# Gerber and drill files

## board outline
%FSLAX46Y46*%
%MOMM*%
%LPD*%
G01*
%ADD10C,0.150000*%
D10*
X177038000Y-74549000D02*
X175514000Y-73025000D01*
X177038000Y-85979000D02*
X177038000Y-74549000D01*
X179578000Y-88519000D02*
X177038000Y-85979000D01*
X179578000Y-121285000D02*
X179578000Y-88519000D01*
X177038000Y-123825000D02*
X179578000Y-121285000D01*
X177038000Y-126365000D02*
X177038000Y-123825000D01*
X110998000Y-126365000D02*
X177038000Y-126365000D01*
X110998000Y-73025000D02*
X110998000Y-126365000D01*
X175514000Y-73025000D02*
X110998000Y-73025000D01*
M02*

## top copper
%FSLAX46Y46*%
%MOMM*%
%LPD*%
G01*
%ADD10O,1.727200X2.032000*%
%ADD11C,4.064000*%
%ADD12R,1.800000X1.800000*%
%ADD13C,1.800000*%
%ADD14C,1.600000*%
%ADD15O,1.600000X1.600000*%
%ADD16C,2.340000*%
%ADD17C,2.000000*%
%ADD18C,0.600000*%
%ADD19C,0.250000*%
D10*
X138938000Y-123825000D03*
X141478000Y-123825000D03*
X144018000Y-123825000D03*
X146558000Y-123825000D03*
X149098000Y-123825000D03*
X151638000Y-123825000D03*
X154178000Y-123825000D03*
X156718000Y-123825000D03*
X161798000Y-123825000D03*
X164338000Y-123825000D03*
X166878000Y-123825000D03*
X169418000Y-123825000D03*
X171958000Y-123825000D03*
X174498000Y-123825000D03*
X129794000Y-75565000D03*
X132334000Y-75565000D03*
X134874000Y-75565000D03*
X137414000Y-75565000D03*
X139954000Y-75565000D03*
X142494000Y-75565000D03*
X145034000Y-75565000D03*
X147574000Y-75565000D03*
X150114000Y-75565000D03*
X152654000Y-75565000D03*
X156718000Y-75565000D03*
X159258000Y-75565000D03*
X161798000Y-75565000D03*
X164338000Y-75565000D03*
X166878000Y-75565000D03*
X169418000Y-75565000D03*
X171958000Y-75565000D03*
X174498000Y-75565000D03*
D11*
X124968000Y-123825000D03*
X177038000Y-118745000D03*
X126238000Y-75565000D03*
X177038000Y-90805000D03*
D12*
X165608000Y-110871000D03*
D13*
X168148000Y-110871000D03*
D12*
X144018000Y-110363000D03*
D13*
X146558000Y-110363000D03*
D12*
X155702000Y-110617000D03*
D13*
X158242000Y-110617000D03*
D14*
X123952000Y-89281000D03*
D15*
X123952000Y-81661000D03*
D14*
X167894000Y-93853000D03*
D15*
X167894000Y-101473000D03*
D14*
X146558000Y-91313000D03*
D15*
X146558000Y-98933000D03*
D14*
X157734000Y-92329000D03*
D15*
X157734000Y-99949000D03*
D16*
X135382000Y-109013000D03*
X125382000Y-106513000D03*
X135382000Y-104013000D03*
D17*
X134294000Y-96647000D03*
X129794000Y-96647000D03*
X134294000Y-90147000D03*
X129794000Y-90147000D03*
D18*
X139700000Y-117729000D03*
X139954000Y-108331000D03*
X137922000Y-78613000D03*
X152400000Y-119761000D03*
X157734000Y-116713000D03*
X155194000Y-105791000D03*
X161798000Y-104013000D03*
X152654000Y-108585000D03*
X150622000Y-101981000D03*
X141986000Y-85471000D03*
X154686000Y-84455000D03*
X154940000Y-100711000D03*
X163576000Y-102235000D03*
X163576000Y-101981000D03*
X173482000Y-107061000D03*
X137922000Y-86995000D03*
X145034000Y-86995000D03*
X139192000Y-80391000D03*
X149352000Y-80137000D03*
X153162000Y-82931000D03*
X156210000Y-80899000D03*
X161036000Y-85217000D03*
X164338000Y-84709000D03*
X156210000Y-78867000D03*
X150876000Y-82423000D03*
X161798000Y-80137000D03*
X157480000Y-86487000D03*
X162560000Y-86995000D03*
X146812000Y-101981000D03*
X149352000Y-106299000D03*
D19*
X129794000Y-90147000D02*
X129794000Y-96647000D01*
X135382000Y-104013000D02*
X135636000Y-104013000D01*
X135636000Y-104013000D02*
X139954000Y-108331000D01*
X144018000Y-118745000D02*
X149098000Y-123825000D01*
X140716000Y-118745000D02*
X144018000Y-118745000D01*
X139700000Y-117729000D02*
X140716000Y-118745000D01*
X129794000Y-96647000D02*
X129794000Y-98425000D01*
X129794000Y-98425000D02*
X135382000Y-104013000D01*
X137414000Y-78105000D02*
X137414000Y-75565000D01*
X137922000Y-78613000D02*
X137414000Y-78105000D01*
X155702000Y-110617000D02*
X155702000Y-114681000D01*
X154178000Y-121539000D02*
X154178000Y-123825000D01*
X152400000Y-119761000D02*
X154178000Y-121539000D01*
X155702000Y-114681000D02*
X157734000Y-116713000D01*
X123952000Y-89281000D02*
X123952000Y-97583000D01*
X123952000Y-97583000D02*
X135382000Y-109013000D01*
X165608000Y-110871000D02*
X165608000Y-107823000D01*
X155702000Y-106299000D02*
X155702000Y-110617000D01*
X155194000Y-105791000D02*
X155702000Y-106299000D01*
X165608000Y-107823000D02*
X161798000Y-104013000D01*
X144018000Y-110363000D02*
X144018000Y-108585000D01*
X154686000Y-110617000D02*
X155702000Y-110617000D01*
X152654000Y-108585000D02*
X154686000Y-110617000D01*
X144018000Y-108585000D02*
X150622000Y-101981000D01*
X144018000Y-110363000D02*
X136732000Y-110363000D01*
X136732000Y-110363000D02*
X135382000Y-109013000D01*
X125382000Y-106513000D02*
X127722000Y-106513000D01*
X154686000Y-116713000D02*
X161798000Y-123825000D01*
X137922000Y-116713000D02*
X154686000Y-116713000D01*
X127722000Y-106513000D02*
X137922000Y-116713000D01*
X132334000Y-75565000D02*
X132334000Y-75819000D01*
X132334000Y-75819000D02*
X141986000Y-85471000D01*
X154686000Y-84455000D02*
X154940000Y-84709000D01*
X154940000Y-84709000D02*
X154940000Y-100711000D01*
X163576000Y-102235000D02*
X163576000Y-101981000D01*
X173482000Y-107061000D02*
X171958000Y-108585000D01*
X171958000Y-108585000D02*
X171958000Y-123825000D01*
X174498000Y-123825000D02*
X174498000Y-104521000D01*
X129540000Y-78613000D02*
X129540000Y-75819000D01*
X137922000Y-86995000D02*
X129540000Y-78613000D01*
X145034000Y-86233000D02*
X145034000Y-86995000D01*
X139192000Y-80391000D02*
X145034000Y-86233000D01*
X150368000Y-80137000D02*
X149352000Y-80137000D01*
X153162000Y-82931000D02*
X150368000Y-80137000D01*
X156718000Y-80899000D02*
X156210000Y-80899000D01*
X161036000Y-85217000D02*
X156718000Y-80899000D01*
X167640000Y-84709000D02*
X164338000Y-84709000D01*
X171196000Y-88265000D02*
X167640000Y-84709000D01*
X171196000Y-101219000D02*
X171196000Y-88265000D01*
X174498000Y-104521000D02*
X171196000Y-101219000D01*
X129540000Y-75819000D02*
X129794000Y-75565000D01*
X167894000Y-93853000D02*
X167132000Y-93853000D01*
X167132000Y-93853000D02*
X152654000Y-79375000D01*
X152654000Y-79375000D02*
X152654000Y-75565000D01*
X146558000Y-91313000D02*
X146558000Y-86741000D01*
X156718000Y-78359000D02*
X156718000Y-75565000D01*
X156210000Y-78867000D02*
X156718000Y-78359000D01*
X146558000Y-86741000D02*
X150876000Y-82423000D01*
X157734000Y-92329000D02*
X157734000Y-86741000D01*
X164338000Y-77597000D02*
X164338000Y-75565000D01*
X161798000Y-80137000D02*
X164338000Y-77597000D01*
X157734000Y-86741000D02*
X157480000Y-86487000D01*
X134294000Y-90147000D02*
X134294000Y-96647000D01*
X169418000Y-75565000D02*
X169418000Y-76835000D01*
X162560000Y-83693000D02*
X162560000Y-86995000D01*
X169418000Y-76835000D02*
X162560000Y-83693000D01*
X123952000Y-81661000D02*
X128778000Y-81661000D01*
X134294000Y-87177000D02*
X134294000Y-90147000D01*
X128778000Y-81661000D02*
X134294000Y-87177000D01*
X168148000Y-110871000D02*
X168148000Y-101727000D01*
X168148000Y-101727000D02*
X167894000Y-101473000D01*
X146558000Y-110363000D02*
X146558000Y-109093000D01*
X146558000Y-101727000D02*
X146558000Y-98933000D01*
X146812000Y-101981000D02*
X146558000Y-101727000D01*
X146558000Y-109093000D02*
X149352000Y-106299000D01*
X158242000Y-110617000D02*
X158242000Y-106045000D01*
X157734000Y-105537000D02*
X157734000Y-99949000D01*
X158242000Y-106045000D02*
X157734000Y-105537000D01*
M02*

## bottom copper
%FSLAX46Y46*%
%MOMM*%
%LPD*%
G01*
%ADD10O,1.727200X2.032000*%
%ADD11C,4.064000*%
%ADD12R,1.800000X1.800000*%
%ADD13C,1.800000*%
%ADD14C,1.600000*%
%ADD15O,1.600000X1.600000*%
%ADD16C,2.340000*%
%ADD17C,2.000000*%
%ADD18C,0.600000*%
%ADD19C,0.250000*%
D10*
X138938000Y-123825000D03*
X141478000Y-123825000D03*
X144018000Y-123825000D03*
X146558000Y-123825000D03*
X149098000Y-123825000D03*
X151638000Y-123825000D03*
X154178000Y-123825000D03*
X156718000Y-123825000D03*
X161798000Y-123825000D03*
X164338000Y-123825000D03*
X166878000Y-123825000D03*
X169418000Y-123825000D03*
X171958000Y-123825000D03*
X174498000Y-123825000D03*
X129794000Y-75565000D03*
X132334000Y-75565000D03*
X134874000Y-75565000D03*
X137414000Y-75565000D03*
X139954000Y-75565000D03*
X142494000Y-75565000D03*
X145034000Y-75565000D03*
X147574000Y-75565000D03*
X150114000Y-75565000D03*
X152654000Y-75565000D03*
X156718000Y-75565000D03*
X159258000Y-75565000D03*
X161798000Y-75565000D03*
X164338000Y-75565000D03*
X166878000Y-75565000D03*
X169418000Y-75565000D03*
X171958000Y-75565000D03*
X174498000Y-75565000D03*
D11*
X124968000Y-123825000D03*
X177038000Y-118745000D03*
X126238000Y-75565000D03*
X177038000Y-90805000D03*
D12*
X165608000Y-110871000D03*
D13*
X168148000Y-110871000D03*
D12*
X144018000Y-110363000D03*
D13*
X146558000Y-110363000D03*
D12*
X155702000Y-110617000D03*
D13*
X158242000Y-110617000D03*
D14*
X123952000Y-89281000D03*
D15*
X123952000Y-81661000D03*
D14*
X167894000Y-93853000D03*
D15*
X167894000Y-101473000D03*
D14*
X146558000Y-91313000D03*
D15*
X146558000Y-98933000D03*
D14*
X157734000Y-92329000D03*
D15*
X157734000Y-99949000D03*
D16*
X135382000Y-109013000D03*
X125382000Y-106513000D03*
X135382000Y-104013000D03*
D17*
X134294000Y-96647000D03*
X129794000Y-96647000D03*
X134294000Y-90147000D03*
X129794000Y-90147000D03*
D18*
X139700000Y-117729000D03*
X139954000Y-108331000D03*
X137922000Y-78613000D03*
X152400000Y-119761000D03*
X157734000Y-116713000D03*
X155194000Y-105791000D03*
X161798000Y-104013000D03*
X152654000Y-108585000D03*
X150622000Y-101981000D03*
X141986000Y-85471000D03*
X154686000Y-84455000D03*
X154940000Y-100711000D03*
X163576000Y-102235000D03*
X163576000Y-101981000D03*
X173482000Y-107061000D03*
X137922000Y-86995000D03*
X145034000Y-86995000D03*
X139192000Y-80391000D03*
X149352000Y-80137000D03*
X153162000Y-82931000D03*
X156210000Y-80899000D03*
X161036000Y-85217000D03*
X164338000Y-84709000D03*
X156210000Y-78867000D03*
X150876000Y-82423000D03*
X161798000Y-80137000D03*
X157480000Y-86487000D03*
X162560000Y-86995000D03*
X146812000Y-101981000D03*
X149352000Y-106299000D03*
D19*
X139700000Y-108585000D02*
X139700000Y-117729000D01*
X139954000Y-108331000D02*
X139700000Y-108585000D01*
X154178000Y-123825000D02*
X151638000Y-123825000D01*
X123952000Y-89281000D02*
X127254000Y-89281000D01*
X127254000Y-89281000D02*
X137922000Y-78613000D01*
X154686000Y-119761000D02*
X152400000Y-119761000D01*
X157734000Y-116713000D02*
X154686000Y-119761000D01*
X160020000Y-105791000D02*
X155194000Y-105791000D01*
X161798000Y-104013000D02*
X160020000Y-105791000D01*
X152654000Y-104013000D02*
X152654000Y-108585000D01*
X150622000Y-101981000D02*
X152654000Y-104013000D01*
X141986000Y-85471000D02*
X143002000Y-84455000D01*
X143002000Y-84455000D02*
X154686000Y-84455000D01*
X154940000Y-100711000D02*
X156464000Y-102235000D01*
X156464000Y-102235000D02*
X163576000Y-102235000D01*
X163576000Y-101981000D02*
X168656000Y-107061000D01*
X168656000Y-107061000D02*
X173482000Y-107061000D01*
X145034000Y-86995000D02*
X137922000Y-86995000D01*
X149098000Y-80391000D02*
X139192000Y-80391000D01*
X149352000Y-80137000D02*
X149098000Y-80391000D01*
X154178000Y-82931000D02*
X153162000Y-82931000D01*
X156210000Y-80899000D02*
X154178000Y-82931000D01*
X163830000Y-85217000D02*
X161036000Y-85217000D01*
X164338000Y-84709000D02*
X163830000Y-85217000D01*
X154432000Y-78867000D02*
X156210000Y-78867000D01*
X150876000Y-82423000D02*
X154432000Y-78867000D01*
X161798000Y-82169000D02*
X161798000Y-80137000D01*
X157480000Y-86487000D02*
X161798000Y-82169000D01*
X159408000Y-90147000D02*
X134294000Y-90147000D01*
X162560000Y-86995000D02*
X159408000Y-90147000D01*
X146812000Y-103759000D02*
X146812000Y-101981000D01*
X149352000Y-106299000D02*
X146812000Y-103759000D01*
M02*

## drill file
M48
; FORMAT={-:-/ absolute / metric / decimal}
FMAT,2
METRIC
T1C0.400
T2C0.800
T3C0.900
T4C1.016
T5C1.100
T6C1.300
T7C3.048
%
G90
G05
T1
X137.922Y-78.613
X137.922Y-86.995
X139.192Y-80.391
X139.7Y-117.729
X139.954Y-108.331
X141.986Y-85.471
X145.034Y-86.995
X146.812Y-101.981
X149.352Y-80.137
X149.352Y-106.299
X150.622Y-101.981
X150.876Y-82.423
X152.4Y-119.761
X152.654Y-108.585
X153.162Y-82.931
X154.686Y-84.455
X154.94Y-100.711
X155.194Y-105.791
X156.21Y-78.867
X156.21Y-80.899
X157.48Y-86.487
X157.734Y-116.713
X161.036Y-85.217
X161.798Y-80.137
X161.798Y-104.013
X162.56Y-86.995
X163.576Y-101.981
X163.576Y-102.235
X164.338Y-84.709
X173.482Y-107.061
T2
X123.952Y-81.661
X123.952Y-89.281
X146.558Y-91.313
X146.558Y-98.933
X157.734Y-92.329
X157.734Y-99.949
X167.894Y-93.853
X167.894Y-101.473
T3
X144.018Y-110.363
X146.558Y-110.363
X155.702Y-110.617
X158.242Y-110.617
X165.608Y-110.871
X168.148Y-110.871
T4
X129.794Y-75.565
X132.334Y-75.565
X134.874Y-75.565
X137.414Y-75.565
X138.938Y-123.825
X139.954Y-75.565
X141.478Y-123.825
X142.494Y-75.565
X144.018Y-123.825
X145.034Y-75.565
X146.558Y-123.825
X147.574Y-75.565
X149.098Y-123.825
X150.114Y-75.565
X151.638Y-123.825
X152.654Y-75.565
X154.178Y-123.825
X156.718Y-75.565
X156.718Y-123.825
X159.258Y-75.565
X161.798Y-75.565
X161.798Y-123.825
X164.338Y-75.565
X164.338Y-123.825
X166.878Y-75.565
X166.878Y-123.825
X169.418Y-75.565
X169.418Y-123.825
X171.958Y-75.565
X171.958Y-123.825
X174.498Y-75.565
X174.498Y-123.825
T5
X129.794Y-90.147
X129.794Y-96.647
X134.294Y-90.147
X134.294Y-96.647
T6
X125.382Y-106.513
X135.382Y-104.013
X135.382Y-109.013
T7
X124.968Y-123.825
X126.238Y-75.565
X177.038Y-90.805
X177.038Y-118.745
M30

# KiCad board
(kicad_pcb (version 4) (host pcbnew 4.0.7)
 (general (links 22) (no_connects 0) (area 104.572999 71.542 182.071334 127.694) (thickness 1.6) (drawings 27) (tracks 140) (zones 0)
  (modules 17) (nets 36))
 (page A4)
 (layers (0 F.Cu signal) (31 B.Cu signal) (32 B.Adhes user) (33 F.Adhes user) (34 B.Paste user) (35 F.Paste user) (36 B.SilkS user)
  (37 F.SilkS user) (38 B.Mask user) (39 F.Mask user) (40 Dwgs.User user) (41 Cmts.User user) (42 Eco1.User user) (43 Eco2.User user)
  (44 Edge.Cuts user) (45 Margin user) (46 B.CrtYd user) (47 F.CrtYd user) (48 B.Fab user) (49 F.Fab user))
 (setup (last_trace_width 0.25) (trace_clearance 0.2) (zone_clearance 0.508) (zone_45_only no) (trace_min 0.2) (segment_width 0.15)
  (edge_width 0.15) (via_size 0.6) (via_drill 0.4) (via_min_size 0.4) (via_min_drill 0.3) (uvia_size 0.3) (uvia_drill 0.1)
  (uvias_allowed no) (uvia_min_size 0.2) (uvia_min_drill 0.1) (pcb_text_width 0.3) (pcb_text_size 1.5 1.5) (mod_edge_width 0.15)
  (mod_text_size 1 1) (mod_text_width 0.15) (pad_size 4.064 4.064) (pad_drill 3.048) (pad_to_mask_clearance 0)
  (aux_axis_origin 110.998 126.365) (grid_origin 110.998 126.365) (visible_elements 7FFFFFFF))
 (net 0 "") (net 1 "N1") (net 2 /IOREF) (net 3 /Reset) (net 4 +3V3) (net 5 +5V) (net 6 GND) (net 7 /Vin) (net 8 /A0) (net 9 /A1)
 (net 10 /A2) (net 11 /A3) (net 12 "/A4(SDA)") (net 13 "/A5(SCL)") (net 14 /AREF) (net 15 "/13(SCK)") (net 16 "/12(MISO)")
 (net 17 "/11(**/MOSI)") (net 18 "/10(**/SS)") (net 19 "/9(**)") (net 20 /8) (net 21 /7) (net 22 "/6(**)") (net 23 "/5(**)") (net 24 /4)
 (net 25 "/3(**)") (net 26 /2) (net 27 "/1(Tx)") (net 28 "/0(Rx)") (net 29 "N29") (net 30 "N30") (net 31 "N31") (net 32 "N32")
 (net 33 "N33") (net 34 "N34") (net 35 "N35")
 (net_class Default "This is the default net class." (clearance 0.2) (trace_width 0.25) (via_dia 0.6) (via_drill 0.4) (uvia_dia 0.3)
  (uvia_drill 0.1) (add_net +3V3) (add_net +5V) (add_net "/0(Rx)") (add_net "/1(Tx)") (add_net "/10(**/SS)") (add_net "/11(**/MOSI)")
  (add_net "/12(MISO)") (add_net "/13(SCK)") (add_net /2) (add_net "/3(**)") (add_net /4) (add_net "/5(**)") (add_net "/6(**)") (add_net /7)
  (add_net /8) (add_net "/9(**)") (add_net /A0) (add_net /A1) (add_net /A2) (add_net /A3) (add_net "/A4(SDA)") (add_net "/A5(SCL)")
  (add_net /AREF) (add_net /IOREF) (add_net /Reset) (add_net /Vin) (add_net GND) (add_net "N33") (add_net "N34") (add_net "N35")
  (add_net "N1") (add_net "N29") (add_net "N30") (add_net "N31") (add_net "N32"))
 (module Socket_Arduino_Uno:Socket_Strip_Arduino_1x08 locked (layer F.Cu) (at 138.938 123.825)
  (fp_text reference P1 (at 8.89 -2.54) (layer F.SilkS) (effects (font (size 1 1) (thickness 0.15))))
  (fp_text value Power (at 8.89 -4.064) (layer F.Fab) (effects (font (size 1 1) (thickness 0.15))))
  (pad 1 thru_hole oval (at 0 0) (size 1.7272 2.032) (drill 1.016) (layers *.Cu *.Mask F.SilkS) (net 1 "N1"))
  (pad 2 thru_hole oval (at 2.54 0) (size 1.7272 2.032) (drill 1.016) (layers *.Cu *.Mask F.SilkS) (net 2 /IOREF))
  (pad 3 thru_hole oval (at 5.08 0) (size 1.7272 2.032) (drill 1.016) (layers *.Cu *.Mask F.SilkS) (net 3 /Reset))
  (pad 4 thru_hole oval (at 7.62 0) (size 1.7272 2.032) (drill 1.016) (layers *.Cu *.Mask F.SilkS) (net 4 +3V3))
  (pad 5 thru_hole oval (at 10.16 0) (size 1.7272 2.032) (drill 1.016) (layers *.Cu *.Mask F.SilkS) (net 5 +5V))
  (pad 6 thru_hole oval (at 12.7 0) (size 1.7272 2.032) (drill 1.016) (layers *.Cu *.Mask F.SilkS) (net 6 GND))
  (pad 7 thru_hole oval (at 15.24 0) (size 1.7272 2.032) (drill 1.016) (layers *.Cu *.Mask F.SilkS) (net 6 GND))
  (pad 8 thru_hole oval (at 17.78 0) (size 1.7272 2.032) (drill 1.016) (layers *.Cu *.Mask F.SilkS) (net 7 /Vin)))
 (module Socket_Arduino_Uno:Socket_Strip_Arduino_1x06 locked (layer F.Cu) (at 161.798 123.825)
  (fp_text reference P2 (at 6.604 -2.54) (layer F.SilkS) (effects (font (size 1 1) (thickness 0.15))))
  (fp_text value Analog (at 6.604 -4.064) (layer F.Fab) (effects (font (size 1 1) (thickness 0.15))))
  (pad 1 thru_hole oval (at 0 0) (size 1.7272 2.032) (drill 1.016) (layers *.Cu *.Mask F.SilkS) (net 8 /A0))
  (pad 2 thru_hole oval (at 2.54 0) (size 1.7272 2.032) (drill 1.016) (layers *.Cu *.Mask F.SilkS) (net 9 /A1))
  (pad 3 thru_hole oval (at 5.08 0) (size 1.7272 2.032) (drill 1.016) (layers *.Cu *.Mask F.SilkS) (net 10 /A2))
  (pad 4 thru_hole oval (at 7.62 0) (size 1.7272 2.032) (drill 1.016) (layers *.Cu *.Mask F.SilkS) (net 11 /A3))
  (pad 5 thru_hole oval (at 10.16 0) (size 1.7272 2.032) (drill 1.016) (layers *.Cu *.Mask F.SilkS) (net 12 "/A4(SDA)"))
  (pad 6 thru_hole oval (at 12.7 0) (size 1.7272 2.032) (drill 1.016) (layers *.Cu *.Mask F.SilkS) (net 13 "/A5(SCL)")))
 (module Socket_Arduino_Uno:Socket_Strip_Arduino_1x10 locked (layer F.Cu) (at 129.794 75.565)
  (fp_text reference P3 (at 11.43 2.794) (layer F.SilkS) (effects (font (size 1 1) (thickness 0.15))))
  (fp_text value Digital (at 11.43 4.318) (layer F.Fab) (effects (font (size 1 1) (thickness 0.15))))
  (pad 1 thru_hole oval (at 0 0) (size 1.7272 2.032) (drill 1.016) (layers *.Cu *.Mask F.SilkS) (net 13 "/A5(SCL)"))
  (pad 2 thru_hole oval (at 2.54 0) (size 1.7272 2.032) (drill 1.016) (layers *.Cu *.Mask F.SilkS) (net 12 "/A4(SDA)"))
  (pad 3 thru_hole oval (at 5.08 0) (size 1.7272 2.032) (drill 1.016) (layers *.Cu *.Mask F.SilkS) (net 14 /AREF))
  (pad 4 thru_hole oval (at 7.62 0) (size 1.7272 2.032) (drill 1.016) (layers *.Cu *.Mask F.SilkS) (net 6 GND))
  (pad 5 thru_hole oval (at 10.16 0) (size 1.7272 2.032) (drill 1.016) (layers *.Cu *.Mask F.SilkS) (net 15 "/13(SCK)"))
  (pad 6 thru_hole oval (at 12.7 0) (size 1.7272 2.032) (drill 1.016) (layers *.Cu *.Mask F.SilkS) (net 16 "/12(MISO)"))
  (pad 7 thru_hole oval (at 15.24 0) (size 1.7272 2.032) (drill 1.016) (layers *.Cu *.Mask F.SilkS) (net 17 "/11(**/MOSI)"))
  (pad 8 thru_hole oval (at 17.78 0) (size 1.7272 2.032) (drill 1.016) (layers *.Cu *.Mask F.SilkS) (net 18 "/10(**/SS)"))
  (pad 9 thru_hole oval (at 20.32 0) (size 1.7272 2.032) (drill 1.016) (layers *.Cu *.Mask F.SilkS) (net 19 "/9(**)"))
  (pad 10 thru_hole oval (at 22.86 0) (size 1.7272 2.032) (drill 1.016) (layers *.Cu *.Mask F.SilkS) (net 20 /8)))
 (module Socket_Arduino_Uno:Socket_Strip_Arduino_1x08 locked (layer F.Cu) (at 156.718 75.565)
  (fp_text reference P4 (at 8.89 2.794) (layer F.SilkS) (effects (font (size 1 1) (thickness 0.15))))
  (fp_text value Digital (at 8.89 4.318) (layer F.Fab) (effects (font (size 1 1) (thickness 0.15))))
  (pad 1 thru_hole oval (at 0 0) (size 1.7272 2.032) (drill 1.016) (layers *.Cu *.Mask F.SilkS) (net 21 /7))
  (pad 2 thru_hole oval (at 2.54 0) (size 1.7272 2.032) (drill 1.016) (layers *.Cu *.Mask F.SilkS) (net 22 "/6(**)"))
  (pad 3 thru_hole oval (at 5.08 0) (size 1.7272 2.032) (drill 1.016) (layers *.Cu *.Mask F.SilkS) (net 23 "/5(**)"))
  (pad 4 thru_hole oval (at 7.62 0) (size 1.7272 2.032) (drill 1.016) (layers *.Cu *.Mask F.SilkS) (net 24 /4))
  (pad 5 thru_hole oval (at 10.16 0) (size 1.7272 2.032) (drill 1.016) (layers *.Cu *.Mask F.SilkS) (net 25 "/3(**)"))
  (pad 6 thru_hole oval (at 12.7 0) (size 1.7272 2.032) (drill 1.016) (layers *.Cu *.Mask F.SilkS) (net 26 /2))
  (pad 7 thru_hole oval (at 15.24 0) (size 1.7272 2.032) (drill 1.016) (layers *.Cu *.Mask F.SilkS) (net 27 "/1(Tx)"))
  (pad 8 thru_hole oval (at 17.78 0) (size 1.7272 2.032) (drill 1.016) (layers *.Cu *.Mask F.SilkS) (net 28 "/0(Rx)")))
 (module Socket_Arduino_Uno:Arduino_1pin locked (layer F.Cu) (at 124.968 123.825)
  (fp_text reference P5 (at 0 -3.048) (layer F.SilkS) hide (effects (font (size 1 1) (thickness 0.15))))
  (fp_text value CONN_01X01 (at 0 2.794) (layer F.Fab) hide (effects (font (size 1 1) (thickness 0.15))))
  (pad 1 thru_hole circle (at 0 0) (size 4.064 4.064) (drill 3.048) (layers *.Cu *.Mask F.SilkS) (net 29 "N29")))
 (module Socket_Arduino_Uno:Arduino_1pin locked (layer F.Cu) (at 177.038 118.745)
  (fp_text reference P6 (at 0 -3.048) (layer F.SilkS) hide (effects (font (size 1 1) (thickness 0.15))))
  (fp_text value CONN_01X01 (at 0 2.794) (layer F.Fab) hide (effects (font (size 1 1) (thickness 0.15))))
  (pad 1 thru_hole circle (at 0 0) (size 4.064 4.064) (drill 3.048) (layers *.Cu *.Mask F.SilkS) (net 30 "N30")))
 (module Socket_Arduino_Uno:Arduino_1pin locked (layer F.Cu) (at 126.238 75.565)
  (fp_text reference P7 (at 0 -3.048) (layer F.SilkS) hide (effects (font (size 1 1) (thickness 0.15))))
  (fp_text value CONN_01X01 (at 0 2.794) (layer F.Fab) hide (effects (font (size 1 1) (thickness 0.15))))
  (pad 1 thru_hole circle (at 0 0) (size 4.064 4.064) (drill 3.048) (layers *.Cu *.Mask F.SilkS) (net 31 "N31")))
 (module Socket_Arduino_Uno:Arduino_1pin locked (layer F.Cu) (at 177.038 90.805)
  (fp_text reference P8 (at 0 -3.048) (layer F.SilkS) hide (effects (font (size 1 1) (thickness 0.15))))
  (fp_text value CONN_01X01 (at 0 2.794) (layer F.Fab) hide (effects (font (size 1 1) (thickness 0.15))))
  (pad 1 thru_hole circle (at 0 0) (size 4.064 4.064) (drill 3.048) (layers *.Cu *.Mask F.SilkS) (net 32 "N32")))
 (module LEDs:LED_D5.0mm (layer F.Cu) (at 165.608 110.871)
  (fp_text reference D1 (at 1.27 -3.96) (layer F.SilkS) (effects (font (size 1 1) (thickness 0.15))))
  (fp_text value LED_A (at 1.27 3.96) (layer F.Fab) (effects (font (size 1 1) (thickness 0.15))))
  (pad 1 thru_hole rect (at 0 0) (size 1.8 1.8) (drill 0.9) (layers *.Cu *.Mask) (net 6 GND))
  (pad 2 thru_hole circle (at 2.54 0) (size 1.8 1.8) (drill 0.9) (layers *.Cu *.Mask) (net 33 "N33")))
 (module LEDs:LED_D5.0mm (layer F.Cu) (at 144.018 110.363)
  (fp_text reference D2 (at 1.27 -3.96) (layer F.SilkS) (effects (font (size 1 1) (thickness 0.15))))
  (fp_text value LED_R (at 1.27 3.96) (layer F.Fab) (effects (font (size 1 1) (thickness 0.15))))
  (pad 1 thru_hole rect (at 0 0) (size 1.8 1.8) (drill 0.9) (layers *.Cu *.Mask) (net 6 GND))
  (pad 2 thru_hole circle (at 2.54 0) (size 1.8 1.8) (drill 0.9) (layers *.Cu *.Mask) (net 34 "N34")))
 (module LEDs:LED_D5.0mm (layer F.Cu) (at 155.702 110.617)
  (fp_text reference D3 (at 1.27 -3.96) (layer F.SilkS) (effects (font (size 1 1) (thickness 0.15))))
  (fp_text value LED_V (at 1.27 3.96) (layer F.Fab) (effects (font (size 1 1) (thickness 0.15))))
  (pad 1 thru_hole rect (at 0 0) (size 1.8 1.8) (drill 0.9) (layers *.Cu *.Mask) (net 6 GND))
  (pad 2 thru_hole circle (at 2.54 0) (size 1.8 1.8) (drill 0.9) (layers *.Cu *.Mask) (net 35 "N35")))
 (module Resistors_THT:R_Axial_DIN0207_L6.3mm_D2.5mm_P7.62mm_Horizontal (layer F.Cu) (at 123.952 89.281 90)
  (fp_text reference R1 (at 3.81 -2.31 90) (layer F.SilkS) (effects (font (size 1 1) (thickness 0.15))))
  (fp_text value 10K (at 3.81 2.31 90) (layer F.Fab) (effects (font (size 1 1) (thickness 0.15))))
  (pad 1 thru_hole circle (at 0 0 90) (size 1.6 1.6) (drill 0.8) (layers *.Cu *.Mask) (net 6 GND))
  (pad 2 thru_hole oval (at 7.62 0 90) (size 1.6 1.6) (drill 0.8) (layers *.Cu *.Mask) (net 26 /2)))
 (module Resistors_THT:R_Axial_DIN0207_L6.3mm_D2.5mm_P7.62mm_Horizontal (layer F.Cu) (at 167.894 93.853 270)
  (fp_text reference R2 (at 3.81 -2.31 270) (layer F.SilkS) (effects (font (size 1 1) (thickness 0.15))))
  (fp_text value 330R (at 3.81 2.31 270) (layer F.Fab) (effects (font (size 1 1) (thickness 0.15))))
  (pad 1 thru_hole circle (at 0 0 270) (size 1.6 1.6) (drill 0.8) (layers *.Cu *.Mask) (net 20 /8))
  (pad 2 thru_hole oval (at 7.62 0 270) (size 1.6 1.6) (drill 0.8) (layers *.Cu *.Mask) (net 33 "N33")))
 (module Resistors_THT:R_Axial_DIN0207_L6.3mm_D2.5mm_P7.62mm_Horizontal (layer F.Cu) (at 146.558 91.313 270)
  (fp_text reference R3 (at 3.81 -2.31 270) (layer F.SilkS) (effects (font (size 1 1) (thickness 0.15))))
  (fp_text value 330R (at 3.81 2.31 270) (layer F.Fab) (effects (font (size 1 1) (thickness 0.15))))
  (pad 1 thru_hole circle (at 0 0 270) (size 1.6 1.6) (drill 0.8) (layers *.Cu *.Mask) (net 21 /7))
  (pad 2 thru_hole oval (at 7.62 0 270) (size 1.6 1.6) (drill 0.8) (layers *.Cu *.Mask) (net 34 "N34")))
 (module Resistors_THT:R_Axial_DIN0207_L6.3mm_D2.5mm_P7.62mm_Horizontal (layer F.Cu) (at 157.734 92.329 270)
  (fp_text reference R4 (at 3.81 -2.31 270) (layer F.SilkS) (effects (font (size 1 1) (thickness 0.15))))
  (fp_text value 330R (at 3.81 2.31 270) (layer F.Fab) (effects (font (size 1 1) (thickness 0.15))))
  (pad 1 thru_hole circle (at 0 0 270) (size 1.6 1.6) (drill 0.8) (layers *.Cu *.Mask) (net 24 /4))
  (pad 2 thru_hole oval (at 7.62 0 270) (size 1.6 1.6) (drill 0.8) (layers *.Cu *.Mask) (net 35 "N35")))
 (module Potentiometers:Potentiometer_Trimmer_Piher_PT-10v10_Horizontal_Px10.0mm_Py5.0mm (layer F.Cu) (at 135.382 104.013 180)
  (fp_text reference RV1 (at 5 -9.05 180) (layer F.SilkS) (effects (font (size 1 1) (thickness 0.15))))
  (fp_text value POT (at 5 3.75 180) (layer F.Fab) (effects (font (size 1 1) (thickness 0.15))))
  (pad 3 thru_hole circle (at 0 -5 180) (size 2.34 2.34) (drill 1.3) (layers *.Cu *.Mask) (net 6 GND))
  (pad 2 thru_hole circle (at 10 -2.5 180) (size 2.34 2.34) (drill 1.3) (layers *.Cu *.Mask) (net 8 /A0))
  (pad 1 thru_hole circle (at 0 0 180) (size 2.34 2.34) (drill 1.3) (layers *.Cu *.Mask) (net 5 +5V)))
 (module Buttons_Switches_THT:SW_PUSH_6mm (layer F.Cu) (at 129.794 96.647 90)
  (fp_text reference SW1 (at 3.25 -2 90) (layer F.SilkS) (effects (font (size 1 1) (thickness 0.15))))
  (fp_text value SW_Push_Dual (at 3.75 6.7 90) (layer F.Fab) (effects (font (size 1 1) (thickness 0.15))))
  (pad 2 thru_hole circle (at 0 4.5 180) (size 2 2) (drill 1.1) (layers *.Cu *.Mask) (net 26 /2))
  (pad 1 thru_hole circle (at 0 0 180) (size 2 2) (drill 1.1) (layers *.Cu *.Mask) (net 5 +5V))
  (pad 2 thru_hole circle (at 6.5 4.5 180) (size 2 2) (drill 1.1) (layers *.Cu *.Mask) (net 26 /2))
  (pad 1 thru_hole circle (at 6.5 0 180) (size 2 2) (drill 1.1) (layers *.Cu *.Mask) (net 5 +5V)))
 (gr_line (start 177.038 74.549) (end 175.514 73.025) (angle 90) (layer Edge.Cuts) (width 0.15))
 (gr_line (start 177.038 85.979) (end 177.038 74.549) (angle 90) (layer Edge.Cuts) (width 0.15))
 (gr_line (start 179.578 88.519) (end 177.038 85.979) (angle 90) (layer Edge.Cuts) (width 0.15))
 (gr_line (start 179.578 121.285) (end 179.578 88.519) (angle 90) (layer Edge.Cuts) (width 0.15))
 (gr_line (start 177.038 123.825) (end 179.578 121.285) (angle 90) (layer Edge.Cuts) (width 0.15))
 (gr_line (start 177.038 126.365) (end 177.038 123.825) (angle 90) (layer Edge.Cuts) (width 0.15))
 (gr_line (start 110.998 126.365) (end 177.038 126.365) (angle 90) (layer Edge.Cuts) (width 0.15))
 (gr_line (start 110.998 73.025) (end 110.998 126.365) (angle 90) (layer Edge.Cuts) (width 0.15))
 (gr_line (start 175.514 73.025) (end 110.998 73.025) (angle 90) (layer Edge.Cuts) (width 0.15))
 (segment (start 129.794 90.147) (end 129.794 96.647) (width 0.25) (layer F.Cu) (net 5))
 (segment (start 135.382 104.013) (end 135.636 104.013) (width 0.25) (layer F.Cu) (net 5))
 (segment (start 135.636 104.013) (end 139.954 108.331) (width 0.25) (layer F.Cu) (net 5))
 (segment (start 144.018 118.745) (end 149.098 123.825) (width 0.25) (layer F.Cu) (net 5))
 (segment (start 140.716 118.745) (end 144.018 118.745) (width 0.25) (layer F.Cu) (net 5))
 (segment (start 139.7 117.729) (end 140.716 118.745) (width 0.25) (layer F.Cu) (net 5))
 (via (at 139.7 117.729) (size 0.6) (drill 0.4) (layers F.Cu B.Cu) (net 5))
 (segment (start 139.7 108.585) (end 139.7 117.729) (width 0.25) (layer B.Cu) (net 5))
 (segment (start 139.954 108.331) (end 139.7 108.585) (width 0.25) (layer B.Cu) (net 5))
 (via (at 139.954 108.331) (size 0.6) (drill 0.4) (layers F.Cu B.Cu) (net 5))
 (segment (start 129.794 96.647) (end 129.794 98.425) (width 0.25) (layer F.Cu) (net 5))
 (segment (start 129.794 98.425) (end 135.382 104.013) (width 0.25) (layer F.Cu) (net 5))
 (segment (start 154.178 123.825) (end 151.638 123.825) (width 0.25) (layer B.Cu) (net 6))
 (segment (start 123.952 89.281) (end 127.254 89.281) (width 0.25) (layer B.Cu) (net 6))
 (segment (start 137.414 78.105) (end 137.414 75.565) (width 0.25) (layer F.Cu) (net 6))
 (segment (start 137.922 78.613) (end 137.414 78.105) (width 0.25) (layer F.Cu) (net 6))
 (via (at 137.922 78.613) (size 0.6) (drill 0.4) (layers F.Cu B.Cu) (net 6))
 (segment (start 127.254 89.281) (end 137.922 78.613) (width 0.25) (layer B.Cu) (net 6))
 (segment (start 155.702 110.617) (end 155.702 114.681) (width 0.25) (layer F.Cu) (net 6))
 (segment (start 154.178 121.539) (end 154.178 123.825) (width 0.25) (layer F.Cu) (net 6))
 (segment (start 152.4 119.761) (end 154.178 121.539) (width 0.25) (layer F.Cu) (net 6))
 (via (at 152.4 119.761) (size 0.6) (drill 0.4) (layers F.Cu B.Cu) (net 6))
 (segment (start 154.686 119.761) (end 152.4 119.761) (width 0.25) (layer B.Cu) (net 6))
 (segment (start 157.734 116.713) (end 154.686 119.761) (width 0.25) (layer B.Cu) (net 6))
 (via (at 157.734 116.713) (size 0.6) (drill 0.4) (layers F.Cu B.Cu) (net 6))
 (segment (start 155.702 114.681) (end 157.734 116.713) (width 0.25) (layer F.Cu) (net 6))
 (segment (start 123.952 89.281) (end 123.952 97.583) (width 0.25) (layer F.Cu) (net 6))
 (segment (start 123.952 97.583) (end 135.382 109.013) (width 0.25) (layer F.Cu) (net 6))
 (segment (start 165.608 110.871) (end 165.608 107.823) (width 0.25) (layer F.Cu) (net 6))
 (segment (start 155.702 106.299) (end 155.702 110.617) (width 0.25) (layer F.Cu) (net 6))
 (segment (start 155.194 105.791) (end 155.702 106.299) (width 0.25) (layer F.Cu) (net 6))
 (via (at 155.194 105.791) (size 0.6) (drill 0.4) (layers F.Cu B.Cu) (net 6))
 (segment (start 160.02 105.791) (end 155.194 105.791) (width 0.25) (layer B.Cu) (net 6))
 (segment (start 161.798 104.013) (end 160.02 105.791) (width 0.25) (layer B.Cu) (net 6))
 (via (at 161.798 104.013) (size 0.6) (drill 0.4) (layers F.Cu B.Cu) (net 6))
 (segment (start 165.608 107.823) (end 161.798 104.013) (width 0.25) (layer F.Cu) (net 6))
 (segment (start 144.018 110.363) (end 144.018 108.585) (width 0.25) (layer F.Cu) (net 6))
 (segment (start 154.686 110.617) (end 155.702 110.617) (width 0.25) (layer F.Cu) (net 6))
 (segment (start 152.654 108.585) (end 154.686 110.617) (width 0.25) (layer F.Cu) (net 6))
 (via (at 152.654 108.585) (size 0.6) (drill 0.4) (layers F.Cu B.Cu) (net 6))
 (segment (start 152.654 104.013) (end 152.654 108.585) (width 0.25) (layer B.Cu) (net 6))
 (segment (start 150.622 101.981) (end 152.654 104.013) (width 0.25) (layer B.Cu) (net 6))
 (via (at 150.622 101.981) (size 0.6) (drill 0.4) (layers F.Cu B.Cu) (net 6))
 (segment (start 144.018 108.585) (end 150.622 101.981) (width 0.25) (layer F.Cu) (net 6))
 (segment (start 144.018 110.363) (end 136.732 110.363) (width 0.25) (layer F.Cu) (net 6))
 (segment (start 136.732 110.363) (end 135.382 109.013) (width 0.25) (layer F.Cu) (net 6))
 (segment (start 125.382 106.513) (end 127.722 106.513) (width 0.25) (layer F.Cu) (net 8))
 (segment (start 154.686 116.713) (end 161.798 123.825) (width 0.25) (layer F.Cu) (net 8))
 (segment (start 137.922 116.713) (end 154.686 116.713) (width 0.25) (layer F.Cu) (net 8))
 (segment (start 127.722 106.513) (end 137.922 116.713) (width 0.25) (layer F.Cu) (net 8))
 (segment (start 132.334 75.565) (end 132.334 75.819) (width 0.25) (layer F.Cu) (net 12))
 (segment (start 132.334 75.819) (end 141.986 85.471) (width 0.25) (layer F.Cu) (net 12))
 (via (at 141.986 85.471) (size 0.6) (drill 0.4) (layers F.Cu B.Cu) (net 12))
 (segment (start 141.986 85.471) (end 143.002 84.455) (width 0.25) (layer B.Cu) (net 12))
 (segment (start 143.002 84.455) (end 154.686 84.455) (width 0.25) (layer B.Cu) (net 12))
 (via (at 154.686 84.455) (size 0.6) (drill 0.4) (layers F.Cu B.Cu) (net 12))
 (segment (start 154.686 84.455) (end 154.94 84.709) (width 0.25) (layer F.Cu) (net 12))
 (segment (start 154.94 84.709) (end 154.94 100.711) (width 0.25) (layer F.Cu) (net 12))
 (via (at 154.94 100.711) (size 0.6) (drill 0.4) (layers F.Cu B.Cu) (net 12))
 (segment (start 154.94 100.711) (end 156.464 102.235) (width 0.25) (layer B.Cu) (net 12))
 (segment (start 156.464 102.235) (end 163.576 102.235) (width 0.25) (layer B.Cu) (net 12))
 (via (at 163.576 102.235) (size 0.6) (drill 0.4) (layers F.Cu B.Cu) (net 12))
 (segment (start 163.576 102.235) (end 163.576 101.981) (width 0.25) (layer F.Cu) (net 12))
 (via (at 163.576 101.981) (size 0.6) (drill 0.4) (layers F.Cu B.Cu) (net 12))
 (segment (start 163.576 101.981) (end 168.656 107.061) (width 0.25) (layer B.Cu) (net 12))
 (segment (start 168.656 107.061) (end 173.482 107.061) (width 0.25) (layer B.Cu) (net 12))
 (via (at 173.482 107.061) (size 0.6) (drill 0.4) (layers F.Cu B.Cu) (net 12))
 (segment (start 173.482 107.061) (end 171.958 108.585) (width 0.25) (layer F.Cu) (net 12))
 (segment (start 171.958 108.585) (end 171.958 123.825) (width 0.25) (layer F.Cu) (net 12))
 (segment (start 174.498 123.825) (end 174.498 104.521) (width 0.25) (layer F.Cu) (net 13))
 (segment (start 129.54 78.613) (end 129.54 75.819) (width 0.25) (layer F.Cu) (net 13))
 (segment (start 137.922 86.995) (end 129.54 78.613) (width 0.25) (layer F.Cu) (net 13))
 (via (at 137.922 86.995) (size 0.6) (drill 0.4) (layers F.Cu B.Cu) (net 13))
 (segment (start 145.034 86.995) (end 137.922 86.995) (width 0.25) (layer B.Cu) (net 13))
 (via (at 145.034 86.995) (size 0.6) (drill 0.4) (layers F.Cu B.Cu) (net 13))
 (segment (start 145.034 86.233) (end 145.034 86.995) (width 0.25) (layer F.Cu) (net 13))
 (segment (start 139.192 80.391) (end 145.034 86.233) (width 0.25) (layer F.Cu) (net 13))
 (via (at 139.192 80.391) (size 0.6) (drill 0.4) (layers F.Cu B.Cu) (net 13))
 (segment (start 149.098 80.391) (end 139.192 80.391) (width 0.25) (layer B.Cu) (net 13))
 (segment (start 149.352 80.137) (end 149.098 80.391) (width 0.25) (layer B.Cu) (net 13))
 (via (at 149.352 80.137) (size 0.6) (drill 0.4) (layers F.Cu B.Cu) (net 13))
 (segment (start 150.368 80.137) (end 149.352 80.137) (width 0.25) (layer F.Cu) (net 13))
 (segment (start 153.162 82.931) (end 150.368 80.137) (width 0.25) (layer F.Cu) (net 13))
 (via (at 153.162 82.931) (size 0.6) (drill 0.4) (layers F.Cu B.Cu) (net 13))
 (segment (start 154.178 82.931) (end 153.162 82.931) (width 0.25) (layer B.Cu) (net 13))
 (segment (start 156.21 80.899) (end 154.178 82.931) (width 0.25) (layer B.Cu) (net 13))
 (via (at 156.21 80.899) (size 0.6) (drill 0.4) (layers F.Cu B.Cu) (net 13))
 (segment (start 156.718 80.899) (end 156.21 80.899) (width 0.25) (layer F.Cu) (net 13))
 (segment (start 161.036 85.217) (end 156.718 80.899) (width 0.25) (layer F.Cu) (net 13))
 (via (at 161.036 85.217) (size 0.6) (drill 0.4) (layers F.Cu B.Cu) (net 13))
 (segment (start 163.83 85.217) (end 161.036 85.217) (width 0.25) (layer B.Cu) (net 13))
 (segment (start 164.338 84.709) (end 163.83 85.217) (width 0.25) (layer B.Cu) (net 13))
 (via (at 164.338 84.709) (size 0.6) (drill 0.4) (layers F.Cu B.Cu) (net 13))
 (segment (start 167.64 84.709) (end 164.338 84.709) (width 0.25) (layer F.Cu) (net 13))
 (segment (start 171.196 88.265) (end 167.64 84.709) (width 0.25) (layer F.Cu) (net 13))
 (segment (start 171.196 101.219) (end 171.196 88.265) (width 0.25) (layer F.Cu) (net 13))
 (segment (start 174.498 104.521) (end 171.196 101.219) (width 0.25) (layer F.Cu) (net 13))
 (segment (start 129.54 75.819) (end 129.794 75.565) (width 0.25) (layer F.Cu) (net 13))
 (segment (start 167.894 93.853) (end 167.132 93.853) (width 0.25) (layer F.Cu) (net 20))
 (segment (start 167.132 93.853) (end 152.654 79.375) (width 0.25) (layer F.Cu) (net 20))
 (segment (start 152.654 79.375) (end 152.654 75.565) (width 0.25) (layer F.Cu) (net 20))
 (segment (start 146.558 91.313) (end 146.558 86.741) (width 0.25) (layer F.Cu) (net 21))
 (segment (start 156.718 78.359) (end 156.718 75.565) (width 0.25) (layer F.Cu) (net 21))
 (segment (start 156.21 78.867) (end 156.718 78.359) (width 0.25) (layer F.Cu) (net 21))
 (via (at 156.21 78.867) (size 0.6) (drill 0.4) (layers F.Cu B.Cu) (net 21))
 (segment (start 154.432 78.867) (end 156.21 78.867) (width 0.25) (layer B.Cu) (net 21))
 (segment (start 150.876 82.423) (end 154.432 78.867) (width 0.25) (layer B.Cu) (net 21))
 (via (at 150.876 82.423) (size 0.6) (drill 0.4) (layers F.Cu B.Cu) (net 21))
 (segment (start 146.558 86.741) (end 150.876 82.423) (width 0.25) (layer F.Cu) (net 21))
 (segment (start 157.734 92.329) (end 157.734 86.741) (width 0.25) (layer F.Cu) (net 24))
 (segment (start 164.338 77.597) (end 164.338 75.565) (width 0.25) (layer F.Cu) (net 24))
 (segment (start 161.798 80.137) (end 164.338 77.597) (width 0.25) (layer F.Cu) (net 24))
 (via (at 161.798 80.137) (size 0.6) (drill 0.4) (layers F.Cu B.Cu) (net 24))
 (segment (start 161.798 82.169) (end 161.798 80.137) (width 0.25) (layer B.Cu) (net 24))
 (segment (start 157.48 86.487) (end 161.798 82.169) (width 0.25) (layer B.Cu) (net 24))
 (via (at 157.48 86.487) (size 0.6) (drill 0.4) (layers F.Cu B.Cu) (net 24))
 (segment (start 157.734 86.741) (end 157.48 86.487) (width 0.25) (layer F.Cu) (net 24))
 (segment (start 134.294 90.147) (end 134.294 96.647) (width 0.25) (layer F.Cu) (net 26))
 (segment (start 169.418 75.565) (end 169.418 76.835) (width 0.25) (layer F.Cu) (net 26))
 (segment (start 159.408 90.147) (end 134.294 90.147) (width 0.25) (layer B.Cu) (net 26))
 (segment (start 162.56 86.995) (end 159.408 90.147) (width 0.25) (layer B.Cu) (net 26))
 (via (at 162.56 86.995) (size 0.6) (drill 0.4) (layers F.Cu B.Cu) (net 26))
 (segment (start 162.56 83.693) (end 162.56 86.995) (width 0.25) (layer F.Cu) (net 26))
 (segment (start 169.418 76.835) (end 162.56 83.693) (width 0.25) (layer F.Cu) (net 26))
 (segment (start 123.952 81.661) (end 128.778 81.661) (width 0.25) (layer F.Cu) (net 26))
 (segment (start 134.294 87.177) (end 134.294 90.147) (width 0.25) (layer F.Cu) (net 26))
 (segment (start 128.778 81.661) (end 134.294 87.177) (width 0.25) (layer F.Cu) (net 26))
 (segment (start 168.148 110.871) (end 168.148 101.727) (width 0.25) (layer F.Cu) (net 33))
 (segment (start 168.148 101.727) (end 167.894 101.473) (width 0.25) (layer F.Cu) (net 33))
 (segment (start 146.558 110.363) (end 146.558 109.093) (width 0.25) (layer F.Cu) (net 34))
 (segment (start 146.558 101.727) (end 146.558 98.933) (width 0.25) (layer F.Cu) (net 34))
 (segment (start 146.812 101.981) (end 146.558 101.727) (width 0.25) (layer F.Cu) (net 34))
 (via (at 146.812 101.981) (size 0.6) (drill 0.4) (layers F.Cu B.Cu) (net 34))
 (segment (start 146.812 103.759) (end 146.812 101.981) (width 0.25) (layer B.Cu) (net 34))
 (segment (start 149.352 106.299) (end 146.812 103.759) (width 0.25) (layer B.Cu) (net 34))
 (via (at 149.352 106.299) (size 0.6) (drill 0.4) (layers F.Cu B.Cu) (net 34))
 (segment (start 146.558 109.093) (end 149.352 106.299) (width 0.25) (layer F.Cu) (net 34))
 (segment (start 158.242 110.617) (end 158.242 106.045) (width 0.25) (layer F.Cu) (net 35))
 (segment (start 157.734 105.537) (end 157.734 99.949) (width 0.25) (layer F.Cu) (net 35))
 (segment (start 158.242 106.045) (end 157.734 105.537) (width 0.25) (layer F.Cu) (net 35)))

